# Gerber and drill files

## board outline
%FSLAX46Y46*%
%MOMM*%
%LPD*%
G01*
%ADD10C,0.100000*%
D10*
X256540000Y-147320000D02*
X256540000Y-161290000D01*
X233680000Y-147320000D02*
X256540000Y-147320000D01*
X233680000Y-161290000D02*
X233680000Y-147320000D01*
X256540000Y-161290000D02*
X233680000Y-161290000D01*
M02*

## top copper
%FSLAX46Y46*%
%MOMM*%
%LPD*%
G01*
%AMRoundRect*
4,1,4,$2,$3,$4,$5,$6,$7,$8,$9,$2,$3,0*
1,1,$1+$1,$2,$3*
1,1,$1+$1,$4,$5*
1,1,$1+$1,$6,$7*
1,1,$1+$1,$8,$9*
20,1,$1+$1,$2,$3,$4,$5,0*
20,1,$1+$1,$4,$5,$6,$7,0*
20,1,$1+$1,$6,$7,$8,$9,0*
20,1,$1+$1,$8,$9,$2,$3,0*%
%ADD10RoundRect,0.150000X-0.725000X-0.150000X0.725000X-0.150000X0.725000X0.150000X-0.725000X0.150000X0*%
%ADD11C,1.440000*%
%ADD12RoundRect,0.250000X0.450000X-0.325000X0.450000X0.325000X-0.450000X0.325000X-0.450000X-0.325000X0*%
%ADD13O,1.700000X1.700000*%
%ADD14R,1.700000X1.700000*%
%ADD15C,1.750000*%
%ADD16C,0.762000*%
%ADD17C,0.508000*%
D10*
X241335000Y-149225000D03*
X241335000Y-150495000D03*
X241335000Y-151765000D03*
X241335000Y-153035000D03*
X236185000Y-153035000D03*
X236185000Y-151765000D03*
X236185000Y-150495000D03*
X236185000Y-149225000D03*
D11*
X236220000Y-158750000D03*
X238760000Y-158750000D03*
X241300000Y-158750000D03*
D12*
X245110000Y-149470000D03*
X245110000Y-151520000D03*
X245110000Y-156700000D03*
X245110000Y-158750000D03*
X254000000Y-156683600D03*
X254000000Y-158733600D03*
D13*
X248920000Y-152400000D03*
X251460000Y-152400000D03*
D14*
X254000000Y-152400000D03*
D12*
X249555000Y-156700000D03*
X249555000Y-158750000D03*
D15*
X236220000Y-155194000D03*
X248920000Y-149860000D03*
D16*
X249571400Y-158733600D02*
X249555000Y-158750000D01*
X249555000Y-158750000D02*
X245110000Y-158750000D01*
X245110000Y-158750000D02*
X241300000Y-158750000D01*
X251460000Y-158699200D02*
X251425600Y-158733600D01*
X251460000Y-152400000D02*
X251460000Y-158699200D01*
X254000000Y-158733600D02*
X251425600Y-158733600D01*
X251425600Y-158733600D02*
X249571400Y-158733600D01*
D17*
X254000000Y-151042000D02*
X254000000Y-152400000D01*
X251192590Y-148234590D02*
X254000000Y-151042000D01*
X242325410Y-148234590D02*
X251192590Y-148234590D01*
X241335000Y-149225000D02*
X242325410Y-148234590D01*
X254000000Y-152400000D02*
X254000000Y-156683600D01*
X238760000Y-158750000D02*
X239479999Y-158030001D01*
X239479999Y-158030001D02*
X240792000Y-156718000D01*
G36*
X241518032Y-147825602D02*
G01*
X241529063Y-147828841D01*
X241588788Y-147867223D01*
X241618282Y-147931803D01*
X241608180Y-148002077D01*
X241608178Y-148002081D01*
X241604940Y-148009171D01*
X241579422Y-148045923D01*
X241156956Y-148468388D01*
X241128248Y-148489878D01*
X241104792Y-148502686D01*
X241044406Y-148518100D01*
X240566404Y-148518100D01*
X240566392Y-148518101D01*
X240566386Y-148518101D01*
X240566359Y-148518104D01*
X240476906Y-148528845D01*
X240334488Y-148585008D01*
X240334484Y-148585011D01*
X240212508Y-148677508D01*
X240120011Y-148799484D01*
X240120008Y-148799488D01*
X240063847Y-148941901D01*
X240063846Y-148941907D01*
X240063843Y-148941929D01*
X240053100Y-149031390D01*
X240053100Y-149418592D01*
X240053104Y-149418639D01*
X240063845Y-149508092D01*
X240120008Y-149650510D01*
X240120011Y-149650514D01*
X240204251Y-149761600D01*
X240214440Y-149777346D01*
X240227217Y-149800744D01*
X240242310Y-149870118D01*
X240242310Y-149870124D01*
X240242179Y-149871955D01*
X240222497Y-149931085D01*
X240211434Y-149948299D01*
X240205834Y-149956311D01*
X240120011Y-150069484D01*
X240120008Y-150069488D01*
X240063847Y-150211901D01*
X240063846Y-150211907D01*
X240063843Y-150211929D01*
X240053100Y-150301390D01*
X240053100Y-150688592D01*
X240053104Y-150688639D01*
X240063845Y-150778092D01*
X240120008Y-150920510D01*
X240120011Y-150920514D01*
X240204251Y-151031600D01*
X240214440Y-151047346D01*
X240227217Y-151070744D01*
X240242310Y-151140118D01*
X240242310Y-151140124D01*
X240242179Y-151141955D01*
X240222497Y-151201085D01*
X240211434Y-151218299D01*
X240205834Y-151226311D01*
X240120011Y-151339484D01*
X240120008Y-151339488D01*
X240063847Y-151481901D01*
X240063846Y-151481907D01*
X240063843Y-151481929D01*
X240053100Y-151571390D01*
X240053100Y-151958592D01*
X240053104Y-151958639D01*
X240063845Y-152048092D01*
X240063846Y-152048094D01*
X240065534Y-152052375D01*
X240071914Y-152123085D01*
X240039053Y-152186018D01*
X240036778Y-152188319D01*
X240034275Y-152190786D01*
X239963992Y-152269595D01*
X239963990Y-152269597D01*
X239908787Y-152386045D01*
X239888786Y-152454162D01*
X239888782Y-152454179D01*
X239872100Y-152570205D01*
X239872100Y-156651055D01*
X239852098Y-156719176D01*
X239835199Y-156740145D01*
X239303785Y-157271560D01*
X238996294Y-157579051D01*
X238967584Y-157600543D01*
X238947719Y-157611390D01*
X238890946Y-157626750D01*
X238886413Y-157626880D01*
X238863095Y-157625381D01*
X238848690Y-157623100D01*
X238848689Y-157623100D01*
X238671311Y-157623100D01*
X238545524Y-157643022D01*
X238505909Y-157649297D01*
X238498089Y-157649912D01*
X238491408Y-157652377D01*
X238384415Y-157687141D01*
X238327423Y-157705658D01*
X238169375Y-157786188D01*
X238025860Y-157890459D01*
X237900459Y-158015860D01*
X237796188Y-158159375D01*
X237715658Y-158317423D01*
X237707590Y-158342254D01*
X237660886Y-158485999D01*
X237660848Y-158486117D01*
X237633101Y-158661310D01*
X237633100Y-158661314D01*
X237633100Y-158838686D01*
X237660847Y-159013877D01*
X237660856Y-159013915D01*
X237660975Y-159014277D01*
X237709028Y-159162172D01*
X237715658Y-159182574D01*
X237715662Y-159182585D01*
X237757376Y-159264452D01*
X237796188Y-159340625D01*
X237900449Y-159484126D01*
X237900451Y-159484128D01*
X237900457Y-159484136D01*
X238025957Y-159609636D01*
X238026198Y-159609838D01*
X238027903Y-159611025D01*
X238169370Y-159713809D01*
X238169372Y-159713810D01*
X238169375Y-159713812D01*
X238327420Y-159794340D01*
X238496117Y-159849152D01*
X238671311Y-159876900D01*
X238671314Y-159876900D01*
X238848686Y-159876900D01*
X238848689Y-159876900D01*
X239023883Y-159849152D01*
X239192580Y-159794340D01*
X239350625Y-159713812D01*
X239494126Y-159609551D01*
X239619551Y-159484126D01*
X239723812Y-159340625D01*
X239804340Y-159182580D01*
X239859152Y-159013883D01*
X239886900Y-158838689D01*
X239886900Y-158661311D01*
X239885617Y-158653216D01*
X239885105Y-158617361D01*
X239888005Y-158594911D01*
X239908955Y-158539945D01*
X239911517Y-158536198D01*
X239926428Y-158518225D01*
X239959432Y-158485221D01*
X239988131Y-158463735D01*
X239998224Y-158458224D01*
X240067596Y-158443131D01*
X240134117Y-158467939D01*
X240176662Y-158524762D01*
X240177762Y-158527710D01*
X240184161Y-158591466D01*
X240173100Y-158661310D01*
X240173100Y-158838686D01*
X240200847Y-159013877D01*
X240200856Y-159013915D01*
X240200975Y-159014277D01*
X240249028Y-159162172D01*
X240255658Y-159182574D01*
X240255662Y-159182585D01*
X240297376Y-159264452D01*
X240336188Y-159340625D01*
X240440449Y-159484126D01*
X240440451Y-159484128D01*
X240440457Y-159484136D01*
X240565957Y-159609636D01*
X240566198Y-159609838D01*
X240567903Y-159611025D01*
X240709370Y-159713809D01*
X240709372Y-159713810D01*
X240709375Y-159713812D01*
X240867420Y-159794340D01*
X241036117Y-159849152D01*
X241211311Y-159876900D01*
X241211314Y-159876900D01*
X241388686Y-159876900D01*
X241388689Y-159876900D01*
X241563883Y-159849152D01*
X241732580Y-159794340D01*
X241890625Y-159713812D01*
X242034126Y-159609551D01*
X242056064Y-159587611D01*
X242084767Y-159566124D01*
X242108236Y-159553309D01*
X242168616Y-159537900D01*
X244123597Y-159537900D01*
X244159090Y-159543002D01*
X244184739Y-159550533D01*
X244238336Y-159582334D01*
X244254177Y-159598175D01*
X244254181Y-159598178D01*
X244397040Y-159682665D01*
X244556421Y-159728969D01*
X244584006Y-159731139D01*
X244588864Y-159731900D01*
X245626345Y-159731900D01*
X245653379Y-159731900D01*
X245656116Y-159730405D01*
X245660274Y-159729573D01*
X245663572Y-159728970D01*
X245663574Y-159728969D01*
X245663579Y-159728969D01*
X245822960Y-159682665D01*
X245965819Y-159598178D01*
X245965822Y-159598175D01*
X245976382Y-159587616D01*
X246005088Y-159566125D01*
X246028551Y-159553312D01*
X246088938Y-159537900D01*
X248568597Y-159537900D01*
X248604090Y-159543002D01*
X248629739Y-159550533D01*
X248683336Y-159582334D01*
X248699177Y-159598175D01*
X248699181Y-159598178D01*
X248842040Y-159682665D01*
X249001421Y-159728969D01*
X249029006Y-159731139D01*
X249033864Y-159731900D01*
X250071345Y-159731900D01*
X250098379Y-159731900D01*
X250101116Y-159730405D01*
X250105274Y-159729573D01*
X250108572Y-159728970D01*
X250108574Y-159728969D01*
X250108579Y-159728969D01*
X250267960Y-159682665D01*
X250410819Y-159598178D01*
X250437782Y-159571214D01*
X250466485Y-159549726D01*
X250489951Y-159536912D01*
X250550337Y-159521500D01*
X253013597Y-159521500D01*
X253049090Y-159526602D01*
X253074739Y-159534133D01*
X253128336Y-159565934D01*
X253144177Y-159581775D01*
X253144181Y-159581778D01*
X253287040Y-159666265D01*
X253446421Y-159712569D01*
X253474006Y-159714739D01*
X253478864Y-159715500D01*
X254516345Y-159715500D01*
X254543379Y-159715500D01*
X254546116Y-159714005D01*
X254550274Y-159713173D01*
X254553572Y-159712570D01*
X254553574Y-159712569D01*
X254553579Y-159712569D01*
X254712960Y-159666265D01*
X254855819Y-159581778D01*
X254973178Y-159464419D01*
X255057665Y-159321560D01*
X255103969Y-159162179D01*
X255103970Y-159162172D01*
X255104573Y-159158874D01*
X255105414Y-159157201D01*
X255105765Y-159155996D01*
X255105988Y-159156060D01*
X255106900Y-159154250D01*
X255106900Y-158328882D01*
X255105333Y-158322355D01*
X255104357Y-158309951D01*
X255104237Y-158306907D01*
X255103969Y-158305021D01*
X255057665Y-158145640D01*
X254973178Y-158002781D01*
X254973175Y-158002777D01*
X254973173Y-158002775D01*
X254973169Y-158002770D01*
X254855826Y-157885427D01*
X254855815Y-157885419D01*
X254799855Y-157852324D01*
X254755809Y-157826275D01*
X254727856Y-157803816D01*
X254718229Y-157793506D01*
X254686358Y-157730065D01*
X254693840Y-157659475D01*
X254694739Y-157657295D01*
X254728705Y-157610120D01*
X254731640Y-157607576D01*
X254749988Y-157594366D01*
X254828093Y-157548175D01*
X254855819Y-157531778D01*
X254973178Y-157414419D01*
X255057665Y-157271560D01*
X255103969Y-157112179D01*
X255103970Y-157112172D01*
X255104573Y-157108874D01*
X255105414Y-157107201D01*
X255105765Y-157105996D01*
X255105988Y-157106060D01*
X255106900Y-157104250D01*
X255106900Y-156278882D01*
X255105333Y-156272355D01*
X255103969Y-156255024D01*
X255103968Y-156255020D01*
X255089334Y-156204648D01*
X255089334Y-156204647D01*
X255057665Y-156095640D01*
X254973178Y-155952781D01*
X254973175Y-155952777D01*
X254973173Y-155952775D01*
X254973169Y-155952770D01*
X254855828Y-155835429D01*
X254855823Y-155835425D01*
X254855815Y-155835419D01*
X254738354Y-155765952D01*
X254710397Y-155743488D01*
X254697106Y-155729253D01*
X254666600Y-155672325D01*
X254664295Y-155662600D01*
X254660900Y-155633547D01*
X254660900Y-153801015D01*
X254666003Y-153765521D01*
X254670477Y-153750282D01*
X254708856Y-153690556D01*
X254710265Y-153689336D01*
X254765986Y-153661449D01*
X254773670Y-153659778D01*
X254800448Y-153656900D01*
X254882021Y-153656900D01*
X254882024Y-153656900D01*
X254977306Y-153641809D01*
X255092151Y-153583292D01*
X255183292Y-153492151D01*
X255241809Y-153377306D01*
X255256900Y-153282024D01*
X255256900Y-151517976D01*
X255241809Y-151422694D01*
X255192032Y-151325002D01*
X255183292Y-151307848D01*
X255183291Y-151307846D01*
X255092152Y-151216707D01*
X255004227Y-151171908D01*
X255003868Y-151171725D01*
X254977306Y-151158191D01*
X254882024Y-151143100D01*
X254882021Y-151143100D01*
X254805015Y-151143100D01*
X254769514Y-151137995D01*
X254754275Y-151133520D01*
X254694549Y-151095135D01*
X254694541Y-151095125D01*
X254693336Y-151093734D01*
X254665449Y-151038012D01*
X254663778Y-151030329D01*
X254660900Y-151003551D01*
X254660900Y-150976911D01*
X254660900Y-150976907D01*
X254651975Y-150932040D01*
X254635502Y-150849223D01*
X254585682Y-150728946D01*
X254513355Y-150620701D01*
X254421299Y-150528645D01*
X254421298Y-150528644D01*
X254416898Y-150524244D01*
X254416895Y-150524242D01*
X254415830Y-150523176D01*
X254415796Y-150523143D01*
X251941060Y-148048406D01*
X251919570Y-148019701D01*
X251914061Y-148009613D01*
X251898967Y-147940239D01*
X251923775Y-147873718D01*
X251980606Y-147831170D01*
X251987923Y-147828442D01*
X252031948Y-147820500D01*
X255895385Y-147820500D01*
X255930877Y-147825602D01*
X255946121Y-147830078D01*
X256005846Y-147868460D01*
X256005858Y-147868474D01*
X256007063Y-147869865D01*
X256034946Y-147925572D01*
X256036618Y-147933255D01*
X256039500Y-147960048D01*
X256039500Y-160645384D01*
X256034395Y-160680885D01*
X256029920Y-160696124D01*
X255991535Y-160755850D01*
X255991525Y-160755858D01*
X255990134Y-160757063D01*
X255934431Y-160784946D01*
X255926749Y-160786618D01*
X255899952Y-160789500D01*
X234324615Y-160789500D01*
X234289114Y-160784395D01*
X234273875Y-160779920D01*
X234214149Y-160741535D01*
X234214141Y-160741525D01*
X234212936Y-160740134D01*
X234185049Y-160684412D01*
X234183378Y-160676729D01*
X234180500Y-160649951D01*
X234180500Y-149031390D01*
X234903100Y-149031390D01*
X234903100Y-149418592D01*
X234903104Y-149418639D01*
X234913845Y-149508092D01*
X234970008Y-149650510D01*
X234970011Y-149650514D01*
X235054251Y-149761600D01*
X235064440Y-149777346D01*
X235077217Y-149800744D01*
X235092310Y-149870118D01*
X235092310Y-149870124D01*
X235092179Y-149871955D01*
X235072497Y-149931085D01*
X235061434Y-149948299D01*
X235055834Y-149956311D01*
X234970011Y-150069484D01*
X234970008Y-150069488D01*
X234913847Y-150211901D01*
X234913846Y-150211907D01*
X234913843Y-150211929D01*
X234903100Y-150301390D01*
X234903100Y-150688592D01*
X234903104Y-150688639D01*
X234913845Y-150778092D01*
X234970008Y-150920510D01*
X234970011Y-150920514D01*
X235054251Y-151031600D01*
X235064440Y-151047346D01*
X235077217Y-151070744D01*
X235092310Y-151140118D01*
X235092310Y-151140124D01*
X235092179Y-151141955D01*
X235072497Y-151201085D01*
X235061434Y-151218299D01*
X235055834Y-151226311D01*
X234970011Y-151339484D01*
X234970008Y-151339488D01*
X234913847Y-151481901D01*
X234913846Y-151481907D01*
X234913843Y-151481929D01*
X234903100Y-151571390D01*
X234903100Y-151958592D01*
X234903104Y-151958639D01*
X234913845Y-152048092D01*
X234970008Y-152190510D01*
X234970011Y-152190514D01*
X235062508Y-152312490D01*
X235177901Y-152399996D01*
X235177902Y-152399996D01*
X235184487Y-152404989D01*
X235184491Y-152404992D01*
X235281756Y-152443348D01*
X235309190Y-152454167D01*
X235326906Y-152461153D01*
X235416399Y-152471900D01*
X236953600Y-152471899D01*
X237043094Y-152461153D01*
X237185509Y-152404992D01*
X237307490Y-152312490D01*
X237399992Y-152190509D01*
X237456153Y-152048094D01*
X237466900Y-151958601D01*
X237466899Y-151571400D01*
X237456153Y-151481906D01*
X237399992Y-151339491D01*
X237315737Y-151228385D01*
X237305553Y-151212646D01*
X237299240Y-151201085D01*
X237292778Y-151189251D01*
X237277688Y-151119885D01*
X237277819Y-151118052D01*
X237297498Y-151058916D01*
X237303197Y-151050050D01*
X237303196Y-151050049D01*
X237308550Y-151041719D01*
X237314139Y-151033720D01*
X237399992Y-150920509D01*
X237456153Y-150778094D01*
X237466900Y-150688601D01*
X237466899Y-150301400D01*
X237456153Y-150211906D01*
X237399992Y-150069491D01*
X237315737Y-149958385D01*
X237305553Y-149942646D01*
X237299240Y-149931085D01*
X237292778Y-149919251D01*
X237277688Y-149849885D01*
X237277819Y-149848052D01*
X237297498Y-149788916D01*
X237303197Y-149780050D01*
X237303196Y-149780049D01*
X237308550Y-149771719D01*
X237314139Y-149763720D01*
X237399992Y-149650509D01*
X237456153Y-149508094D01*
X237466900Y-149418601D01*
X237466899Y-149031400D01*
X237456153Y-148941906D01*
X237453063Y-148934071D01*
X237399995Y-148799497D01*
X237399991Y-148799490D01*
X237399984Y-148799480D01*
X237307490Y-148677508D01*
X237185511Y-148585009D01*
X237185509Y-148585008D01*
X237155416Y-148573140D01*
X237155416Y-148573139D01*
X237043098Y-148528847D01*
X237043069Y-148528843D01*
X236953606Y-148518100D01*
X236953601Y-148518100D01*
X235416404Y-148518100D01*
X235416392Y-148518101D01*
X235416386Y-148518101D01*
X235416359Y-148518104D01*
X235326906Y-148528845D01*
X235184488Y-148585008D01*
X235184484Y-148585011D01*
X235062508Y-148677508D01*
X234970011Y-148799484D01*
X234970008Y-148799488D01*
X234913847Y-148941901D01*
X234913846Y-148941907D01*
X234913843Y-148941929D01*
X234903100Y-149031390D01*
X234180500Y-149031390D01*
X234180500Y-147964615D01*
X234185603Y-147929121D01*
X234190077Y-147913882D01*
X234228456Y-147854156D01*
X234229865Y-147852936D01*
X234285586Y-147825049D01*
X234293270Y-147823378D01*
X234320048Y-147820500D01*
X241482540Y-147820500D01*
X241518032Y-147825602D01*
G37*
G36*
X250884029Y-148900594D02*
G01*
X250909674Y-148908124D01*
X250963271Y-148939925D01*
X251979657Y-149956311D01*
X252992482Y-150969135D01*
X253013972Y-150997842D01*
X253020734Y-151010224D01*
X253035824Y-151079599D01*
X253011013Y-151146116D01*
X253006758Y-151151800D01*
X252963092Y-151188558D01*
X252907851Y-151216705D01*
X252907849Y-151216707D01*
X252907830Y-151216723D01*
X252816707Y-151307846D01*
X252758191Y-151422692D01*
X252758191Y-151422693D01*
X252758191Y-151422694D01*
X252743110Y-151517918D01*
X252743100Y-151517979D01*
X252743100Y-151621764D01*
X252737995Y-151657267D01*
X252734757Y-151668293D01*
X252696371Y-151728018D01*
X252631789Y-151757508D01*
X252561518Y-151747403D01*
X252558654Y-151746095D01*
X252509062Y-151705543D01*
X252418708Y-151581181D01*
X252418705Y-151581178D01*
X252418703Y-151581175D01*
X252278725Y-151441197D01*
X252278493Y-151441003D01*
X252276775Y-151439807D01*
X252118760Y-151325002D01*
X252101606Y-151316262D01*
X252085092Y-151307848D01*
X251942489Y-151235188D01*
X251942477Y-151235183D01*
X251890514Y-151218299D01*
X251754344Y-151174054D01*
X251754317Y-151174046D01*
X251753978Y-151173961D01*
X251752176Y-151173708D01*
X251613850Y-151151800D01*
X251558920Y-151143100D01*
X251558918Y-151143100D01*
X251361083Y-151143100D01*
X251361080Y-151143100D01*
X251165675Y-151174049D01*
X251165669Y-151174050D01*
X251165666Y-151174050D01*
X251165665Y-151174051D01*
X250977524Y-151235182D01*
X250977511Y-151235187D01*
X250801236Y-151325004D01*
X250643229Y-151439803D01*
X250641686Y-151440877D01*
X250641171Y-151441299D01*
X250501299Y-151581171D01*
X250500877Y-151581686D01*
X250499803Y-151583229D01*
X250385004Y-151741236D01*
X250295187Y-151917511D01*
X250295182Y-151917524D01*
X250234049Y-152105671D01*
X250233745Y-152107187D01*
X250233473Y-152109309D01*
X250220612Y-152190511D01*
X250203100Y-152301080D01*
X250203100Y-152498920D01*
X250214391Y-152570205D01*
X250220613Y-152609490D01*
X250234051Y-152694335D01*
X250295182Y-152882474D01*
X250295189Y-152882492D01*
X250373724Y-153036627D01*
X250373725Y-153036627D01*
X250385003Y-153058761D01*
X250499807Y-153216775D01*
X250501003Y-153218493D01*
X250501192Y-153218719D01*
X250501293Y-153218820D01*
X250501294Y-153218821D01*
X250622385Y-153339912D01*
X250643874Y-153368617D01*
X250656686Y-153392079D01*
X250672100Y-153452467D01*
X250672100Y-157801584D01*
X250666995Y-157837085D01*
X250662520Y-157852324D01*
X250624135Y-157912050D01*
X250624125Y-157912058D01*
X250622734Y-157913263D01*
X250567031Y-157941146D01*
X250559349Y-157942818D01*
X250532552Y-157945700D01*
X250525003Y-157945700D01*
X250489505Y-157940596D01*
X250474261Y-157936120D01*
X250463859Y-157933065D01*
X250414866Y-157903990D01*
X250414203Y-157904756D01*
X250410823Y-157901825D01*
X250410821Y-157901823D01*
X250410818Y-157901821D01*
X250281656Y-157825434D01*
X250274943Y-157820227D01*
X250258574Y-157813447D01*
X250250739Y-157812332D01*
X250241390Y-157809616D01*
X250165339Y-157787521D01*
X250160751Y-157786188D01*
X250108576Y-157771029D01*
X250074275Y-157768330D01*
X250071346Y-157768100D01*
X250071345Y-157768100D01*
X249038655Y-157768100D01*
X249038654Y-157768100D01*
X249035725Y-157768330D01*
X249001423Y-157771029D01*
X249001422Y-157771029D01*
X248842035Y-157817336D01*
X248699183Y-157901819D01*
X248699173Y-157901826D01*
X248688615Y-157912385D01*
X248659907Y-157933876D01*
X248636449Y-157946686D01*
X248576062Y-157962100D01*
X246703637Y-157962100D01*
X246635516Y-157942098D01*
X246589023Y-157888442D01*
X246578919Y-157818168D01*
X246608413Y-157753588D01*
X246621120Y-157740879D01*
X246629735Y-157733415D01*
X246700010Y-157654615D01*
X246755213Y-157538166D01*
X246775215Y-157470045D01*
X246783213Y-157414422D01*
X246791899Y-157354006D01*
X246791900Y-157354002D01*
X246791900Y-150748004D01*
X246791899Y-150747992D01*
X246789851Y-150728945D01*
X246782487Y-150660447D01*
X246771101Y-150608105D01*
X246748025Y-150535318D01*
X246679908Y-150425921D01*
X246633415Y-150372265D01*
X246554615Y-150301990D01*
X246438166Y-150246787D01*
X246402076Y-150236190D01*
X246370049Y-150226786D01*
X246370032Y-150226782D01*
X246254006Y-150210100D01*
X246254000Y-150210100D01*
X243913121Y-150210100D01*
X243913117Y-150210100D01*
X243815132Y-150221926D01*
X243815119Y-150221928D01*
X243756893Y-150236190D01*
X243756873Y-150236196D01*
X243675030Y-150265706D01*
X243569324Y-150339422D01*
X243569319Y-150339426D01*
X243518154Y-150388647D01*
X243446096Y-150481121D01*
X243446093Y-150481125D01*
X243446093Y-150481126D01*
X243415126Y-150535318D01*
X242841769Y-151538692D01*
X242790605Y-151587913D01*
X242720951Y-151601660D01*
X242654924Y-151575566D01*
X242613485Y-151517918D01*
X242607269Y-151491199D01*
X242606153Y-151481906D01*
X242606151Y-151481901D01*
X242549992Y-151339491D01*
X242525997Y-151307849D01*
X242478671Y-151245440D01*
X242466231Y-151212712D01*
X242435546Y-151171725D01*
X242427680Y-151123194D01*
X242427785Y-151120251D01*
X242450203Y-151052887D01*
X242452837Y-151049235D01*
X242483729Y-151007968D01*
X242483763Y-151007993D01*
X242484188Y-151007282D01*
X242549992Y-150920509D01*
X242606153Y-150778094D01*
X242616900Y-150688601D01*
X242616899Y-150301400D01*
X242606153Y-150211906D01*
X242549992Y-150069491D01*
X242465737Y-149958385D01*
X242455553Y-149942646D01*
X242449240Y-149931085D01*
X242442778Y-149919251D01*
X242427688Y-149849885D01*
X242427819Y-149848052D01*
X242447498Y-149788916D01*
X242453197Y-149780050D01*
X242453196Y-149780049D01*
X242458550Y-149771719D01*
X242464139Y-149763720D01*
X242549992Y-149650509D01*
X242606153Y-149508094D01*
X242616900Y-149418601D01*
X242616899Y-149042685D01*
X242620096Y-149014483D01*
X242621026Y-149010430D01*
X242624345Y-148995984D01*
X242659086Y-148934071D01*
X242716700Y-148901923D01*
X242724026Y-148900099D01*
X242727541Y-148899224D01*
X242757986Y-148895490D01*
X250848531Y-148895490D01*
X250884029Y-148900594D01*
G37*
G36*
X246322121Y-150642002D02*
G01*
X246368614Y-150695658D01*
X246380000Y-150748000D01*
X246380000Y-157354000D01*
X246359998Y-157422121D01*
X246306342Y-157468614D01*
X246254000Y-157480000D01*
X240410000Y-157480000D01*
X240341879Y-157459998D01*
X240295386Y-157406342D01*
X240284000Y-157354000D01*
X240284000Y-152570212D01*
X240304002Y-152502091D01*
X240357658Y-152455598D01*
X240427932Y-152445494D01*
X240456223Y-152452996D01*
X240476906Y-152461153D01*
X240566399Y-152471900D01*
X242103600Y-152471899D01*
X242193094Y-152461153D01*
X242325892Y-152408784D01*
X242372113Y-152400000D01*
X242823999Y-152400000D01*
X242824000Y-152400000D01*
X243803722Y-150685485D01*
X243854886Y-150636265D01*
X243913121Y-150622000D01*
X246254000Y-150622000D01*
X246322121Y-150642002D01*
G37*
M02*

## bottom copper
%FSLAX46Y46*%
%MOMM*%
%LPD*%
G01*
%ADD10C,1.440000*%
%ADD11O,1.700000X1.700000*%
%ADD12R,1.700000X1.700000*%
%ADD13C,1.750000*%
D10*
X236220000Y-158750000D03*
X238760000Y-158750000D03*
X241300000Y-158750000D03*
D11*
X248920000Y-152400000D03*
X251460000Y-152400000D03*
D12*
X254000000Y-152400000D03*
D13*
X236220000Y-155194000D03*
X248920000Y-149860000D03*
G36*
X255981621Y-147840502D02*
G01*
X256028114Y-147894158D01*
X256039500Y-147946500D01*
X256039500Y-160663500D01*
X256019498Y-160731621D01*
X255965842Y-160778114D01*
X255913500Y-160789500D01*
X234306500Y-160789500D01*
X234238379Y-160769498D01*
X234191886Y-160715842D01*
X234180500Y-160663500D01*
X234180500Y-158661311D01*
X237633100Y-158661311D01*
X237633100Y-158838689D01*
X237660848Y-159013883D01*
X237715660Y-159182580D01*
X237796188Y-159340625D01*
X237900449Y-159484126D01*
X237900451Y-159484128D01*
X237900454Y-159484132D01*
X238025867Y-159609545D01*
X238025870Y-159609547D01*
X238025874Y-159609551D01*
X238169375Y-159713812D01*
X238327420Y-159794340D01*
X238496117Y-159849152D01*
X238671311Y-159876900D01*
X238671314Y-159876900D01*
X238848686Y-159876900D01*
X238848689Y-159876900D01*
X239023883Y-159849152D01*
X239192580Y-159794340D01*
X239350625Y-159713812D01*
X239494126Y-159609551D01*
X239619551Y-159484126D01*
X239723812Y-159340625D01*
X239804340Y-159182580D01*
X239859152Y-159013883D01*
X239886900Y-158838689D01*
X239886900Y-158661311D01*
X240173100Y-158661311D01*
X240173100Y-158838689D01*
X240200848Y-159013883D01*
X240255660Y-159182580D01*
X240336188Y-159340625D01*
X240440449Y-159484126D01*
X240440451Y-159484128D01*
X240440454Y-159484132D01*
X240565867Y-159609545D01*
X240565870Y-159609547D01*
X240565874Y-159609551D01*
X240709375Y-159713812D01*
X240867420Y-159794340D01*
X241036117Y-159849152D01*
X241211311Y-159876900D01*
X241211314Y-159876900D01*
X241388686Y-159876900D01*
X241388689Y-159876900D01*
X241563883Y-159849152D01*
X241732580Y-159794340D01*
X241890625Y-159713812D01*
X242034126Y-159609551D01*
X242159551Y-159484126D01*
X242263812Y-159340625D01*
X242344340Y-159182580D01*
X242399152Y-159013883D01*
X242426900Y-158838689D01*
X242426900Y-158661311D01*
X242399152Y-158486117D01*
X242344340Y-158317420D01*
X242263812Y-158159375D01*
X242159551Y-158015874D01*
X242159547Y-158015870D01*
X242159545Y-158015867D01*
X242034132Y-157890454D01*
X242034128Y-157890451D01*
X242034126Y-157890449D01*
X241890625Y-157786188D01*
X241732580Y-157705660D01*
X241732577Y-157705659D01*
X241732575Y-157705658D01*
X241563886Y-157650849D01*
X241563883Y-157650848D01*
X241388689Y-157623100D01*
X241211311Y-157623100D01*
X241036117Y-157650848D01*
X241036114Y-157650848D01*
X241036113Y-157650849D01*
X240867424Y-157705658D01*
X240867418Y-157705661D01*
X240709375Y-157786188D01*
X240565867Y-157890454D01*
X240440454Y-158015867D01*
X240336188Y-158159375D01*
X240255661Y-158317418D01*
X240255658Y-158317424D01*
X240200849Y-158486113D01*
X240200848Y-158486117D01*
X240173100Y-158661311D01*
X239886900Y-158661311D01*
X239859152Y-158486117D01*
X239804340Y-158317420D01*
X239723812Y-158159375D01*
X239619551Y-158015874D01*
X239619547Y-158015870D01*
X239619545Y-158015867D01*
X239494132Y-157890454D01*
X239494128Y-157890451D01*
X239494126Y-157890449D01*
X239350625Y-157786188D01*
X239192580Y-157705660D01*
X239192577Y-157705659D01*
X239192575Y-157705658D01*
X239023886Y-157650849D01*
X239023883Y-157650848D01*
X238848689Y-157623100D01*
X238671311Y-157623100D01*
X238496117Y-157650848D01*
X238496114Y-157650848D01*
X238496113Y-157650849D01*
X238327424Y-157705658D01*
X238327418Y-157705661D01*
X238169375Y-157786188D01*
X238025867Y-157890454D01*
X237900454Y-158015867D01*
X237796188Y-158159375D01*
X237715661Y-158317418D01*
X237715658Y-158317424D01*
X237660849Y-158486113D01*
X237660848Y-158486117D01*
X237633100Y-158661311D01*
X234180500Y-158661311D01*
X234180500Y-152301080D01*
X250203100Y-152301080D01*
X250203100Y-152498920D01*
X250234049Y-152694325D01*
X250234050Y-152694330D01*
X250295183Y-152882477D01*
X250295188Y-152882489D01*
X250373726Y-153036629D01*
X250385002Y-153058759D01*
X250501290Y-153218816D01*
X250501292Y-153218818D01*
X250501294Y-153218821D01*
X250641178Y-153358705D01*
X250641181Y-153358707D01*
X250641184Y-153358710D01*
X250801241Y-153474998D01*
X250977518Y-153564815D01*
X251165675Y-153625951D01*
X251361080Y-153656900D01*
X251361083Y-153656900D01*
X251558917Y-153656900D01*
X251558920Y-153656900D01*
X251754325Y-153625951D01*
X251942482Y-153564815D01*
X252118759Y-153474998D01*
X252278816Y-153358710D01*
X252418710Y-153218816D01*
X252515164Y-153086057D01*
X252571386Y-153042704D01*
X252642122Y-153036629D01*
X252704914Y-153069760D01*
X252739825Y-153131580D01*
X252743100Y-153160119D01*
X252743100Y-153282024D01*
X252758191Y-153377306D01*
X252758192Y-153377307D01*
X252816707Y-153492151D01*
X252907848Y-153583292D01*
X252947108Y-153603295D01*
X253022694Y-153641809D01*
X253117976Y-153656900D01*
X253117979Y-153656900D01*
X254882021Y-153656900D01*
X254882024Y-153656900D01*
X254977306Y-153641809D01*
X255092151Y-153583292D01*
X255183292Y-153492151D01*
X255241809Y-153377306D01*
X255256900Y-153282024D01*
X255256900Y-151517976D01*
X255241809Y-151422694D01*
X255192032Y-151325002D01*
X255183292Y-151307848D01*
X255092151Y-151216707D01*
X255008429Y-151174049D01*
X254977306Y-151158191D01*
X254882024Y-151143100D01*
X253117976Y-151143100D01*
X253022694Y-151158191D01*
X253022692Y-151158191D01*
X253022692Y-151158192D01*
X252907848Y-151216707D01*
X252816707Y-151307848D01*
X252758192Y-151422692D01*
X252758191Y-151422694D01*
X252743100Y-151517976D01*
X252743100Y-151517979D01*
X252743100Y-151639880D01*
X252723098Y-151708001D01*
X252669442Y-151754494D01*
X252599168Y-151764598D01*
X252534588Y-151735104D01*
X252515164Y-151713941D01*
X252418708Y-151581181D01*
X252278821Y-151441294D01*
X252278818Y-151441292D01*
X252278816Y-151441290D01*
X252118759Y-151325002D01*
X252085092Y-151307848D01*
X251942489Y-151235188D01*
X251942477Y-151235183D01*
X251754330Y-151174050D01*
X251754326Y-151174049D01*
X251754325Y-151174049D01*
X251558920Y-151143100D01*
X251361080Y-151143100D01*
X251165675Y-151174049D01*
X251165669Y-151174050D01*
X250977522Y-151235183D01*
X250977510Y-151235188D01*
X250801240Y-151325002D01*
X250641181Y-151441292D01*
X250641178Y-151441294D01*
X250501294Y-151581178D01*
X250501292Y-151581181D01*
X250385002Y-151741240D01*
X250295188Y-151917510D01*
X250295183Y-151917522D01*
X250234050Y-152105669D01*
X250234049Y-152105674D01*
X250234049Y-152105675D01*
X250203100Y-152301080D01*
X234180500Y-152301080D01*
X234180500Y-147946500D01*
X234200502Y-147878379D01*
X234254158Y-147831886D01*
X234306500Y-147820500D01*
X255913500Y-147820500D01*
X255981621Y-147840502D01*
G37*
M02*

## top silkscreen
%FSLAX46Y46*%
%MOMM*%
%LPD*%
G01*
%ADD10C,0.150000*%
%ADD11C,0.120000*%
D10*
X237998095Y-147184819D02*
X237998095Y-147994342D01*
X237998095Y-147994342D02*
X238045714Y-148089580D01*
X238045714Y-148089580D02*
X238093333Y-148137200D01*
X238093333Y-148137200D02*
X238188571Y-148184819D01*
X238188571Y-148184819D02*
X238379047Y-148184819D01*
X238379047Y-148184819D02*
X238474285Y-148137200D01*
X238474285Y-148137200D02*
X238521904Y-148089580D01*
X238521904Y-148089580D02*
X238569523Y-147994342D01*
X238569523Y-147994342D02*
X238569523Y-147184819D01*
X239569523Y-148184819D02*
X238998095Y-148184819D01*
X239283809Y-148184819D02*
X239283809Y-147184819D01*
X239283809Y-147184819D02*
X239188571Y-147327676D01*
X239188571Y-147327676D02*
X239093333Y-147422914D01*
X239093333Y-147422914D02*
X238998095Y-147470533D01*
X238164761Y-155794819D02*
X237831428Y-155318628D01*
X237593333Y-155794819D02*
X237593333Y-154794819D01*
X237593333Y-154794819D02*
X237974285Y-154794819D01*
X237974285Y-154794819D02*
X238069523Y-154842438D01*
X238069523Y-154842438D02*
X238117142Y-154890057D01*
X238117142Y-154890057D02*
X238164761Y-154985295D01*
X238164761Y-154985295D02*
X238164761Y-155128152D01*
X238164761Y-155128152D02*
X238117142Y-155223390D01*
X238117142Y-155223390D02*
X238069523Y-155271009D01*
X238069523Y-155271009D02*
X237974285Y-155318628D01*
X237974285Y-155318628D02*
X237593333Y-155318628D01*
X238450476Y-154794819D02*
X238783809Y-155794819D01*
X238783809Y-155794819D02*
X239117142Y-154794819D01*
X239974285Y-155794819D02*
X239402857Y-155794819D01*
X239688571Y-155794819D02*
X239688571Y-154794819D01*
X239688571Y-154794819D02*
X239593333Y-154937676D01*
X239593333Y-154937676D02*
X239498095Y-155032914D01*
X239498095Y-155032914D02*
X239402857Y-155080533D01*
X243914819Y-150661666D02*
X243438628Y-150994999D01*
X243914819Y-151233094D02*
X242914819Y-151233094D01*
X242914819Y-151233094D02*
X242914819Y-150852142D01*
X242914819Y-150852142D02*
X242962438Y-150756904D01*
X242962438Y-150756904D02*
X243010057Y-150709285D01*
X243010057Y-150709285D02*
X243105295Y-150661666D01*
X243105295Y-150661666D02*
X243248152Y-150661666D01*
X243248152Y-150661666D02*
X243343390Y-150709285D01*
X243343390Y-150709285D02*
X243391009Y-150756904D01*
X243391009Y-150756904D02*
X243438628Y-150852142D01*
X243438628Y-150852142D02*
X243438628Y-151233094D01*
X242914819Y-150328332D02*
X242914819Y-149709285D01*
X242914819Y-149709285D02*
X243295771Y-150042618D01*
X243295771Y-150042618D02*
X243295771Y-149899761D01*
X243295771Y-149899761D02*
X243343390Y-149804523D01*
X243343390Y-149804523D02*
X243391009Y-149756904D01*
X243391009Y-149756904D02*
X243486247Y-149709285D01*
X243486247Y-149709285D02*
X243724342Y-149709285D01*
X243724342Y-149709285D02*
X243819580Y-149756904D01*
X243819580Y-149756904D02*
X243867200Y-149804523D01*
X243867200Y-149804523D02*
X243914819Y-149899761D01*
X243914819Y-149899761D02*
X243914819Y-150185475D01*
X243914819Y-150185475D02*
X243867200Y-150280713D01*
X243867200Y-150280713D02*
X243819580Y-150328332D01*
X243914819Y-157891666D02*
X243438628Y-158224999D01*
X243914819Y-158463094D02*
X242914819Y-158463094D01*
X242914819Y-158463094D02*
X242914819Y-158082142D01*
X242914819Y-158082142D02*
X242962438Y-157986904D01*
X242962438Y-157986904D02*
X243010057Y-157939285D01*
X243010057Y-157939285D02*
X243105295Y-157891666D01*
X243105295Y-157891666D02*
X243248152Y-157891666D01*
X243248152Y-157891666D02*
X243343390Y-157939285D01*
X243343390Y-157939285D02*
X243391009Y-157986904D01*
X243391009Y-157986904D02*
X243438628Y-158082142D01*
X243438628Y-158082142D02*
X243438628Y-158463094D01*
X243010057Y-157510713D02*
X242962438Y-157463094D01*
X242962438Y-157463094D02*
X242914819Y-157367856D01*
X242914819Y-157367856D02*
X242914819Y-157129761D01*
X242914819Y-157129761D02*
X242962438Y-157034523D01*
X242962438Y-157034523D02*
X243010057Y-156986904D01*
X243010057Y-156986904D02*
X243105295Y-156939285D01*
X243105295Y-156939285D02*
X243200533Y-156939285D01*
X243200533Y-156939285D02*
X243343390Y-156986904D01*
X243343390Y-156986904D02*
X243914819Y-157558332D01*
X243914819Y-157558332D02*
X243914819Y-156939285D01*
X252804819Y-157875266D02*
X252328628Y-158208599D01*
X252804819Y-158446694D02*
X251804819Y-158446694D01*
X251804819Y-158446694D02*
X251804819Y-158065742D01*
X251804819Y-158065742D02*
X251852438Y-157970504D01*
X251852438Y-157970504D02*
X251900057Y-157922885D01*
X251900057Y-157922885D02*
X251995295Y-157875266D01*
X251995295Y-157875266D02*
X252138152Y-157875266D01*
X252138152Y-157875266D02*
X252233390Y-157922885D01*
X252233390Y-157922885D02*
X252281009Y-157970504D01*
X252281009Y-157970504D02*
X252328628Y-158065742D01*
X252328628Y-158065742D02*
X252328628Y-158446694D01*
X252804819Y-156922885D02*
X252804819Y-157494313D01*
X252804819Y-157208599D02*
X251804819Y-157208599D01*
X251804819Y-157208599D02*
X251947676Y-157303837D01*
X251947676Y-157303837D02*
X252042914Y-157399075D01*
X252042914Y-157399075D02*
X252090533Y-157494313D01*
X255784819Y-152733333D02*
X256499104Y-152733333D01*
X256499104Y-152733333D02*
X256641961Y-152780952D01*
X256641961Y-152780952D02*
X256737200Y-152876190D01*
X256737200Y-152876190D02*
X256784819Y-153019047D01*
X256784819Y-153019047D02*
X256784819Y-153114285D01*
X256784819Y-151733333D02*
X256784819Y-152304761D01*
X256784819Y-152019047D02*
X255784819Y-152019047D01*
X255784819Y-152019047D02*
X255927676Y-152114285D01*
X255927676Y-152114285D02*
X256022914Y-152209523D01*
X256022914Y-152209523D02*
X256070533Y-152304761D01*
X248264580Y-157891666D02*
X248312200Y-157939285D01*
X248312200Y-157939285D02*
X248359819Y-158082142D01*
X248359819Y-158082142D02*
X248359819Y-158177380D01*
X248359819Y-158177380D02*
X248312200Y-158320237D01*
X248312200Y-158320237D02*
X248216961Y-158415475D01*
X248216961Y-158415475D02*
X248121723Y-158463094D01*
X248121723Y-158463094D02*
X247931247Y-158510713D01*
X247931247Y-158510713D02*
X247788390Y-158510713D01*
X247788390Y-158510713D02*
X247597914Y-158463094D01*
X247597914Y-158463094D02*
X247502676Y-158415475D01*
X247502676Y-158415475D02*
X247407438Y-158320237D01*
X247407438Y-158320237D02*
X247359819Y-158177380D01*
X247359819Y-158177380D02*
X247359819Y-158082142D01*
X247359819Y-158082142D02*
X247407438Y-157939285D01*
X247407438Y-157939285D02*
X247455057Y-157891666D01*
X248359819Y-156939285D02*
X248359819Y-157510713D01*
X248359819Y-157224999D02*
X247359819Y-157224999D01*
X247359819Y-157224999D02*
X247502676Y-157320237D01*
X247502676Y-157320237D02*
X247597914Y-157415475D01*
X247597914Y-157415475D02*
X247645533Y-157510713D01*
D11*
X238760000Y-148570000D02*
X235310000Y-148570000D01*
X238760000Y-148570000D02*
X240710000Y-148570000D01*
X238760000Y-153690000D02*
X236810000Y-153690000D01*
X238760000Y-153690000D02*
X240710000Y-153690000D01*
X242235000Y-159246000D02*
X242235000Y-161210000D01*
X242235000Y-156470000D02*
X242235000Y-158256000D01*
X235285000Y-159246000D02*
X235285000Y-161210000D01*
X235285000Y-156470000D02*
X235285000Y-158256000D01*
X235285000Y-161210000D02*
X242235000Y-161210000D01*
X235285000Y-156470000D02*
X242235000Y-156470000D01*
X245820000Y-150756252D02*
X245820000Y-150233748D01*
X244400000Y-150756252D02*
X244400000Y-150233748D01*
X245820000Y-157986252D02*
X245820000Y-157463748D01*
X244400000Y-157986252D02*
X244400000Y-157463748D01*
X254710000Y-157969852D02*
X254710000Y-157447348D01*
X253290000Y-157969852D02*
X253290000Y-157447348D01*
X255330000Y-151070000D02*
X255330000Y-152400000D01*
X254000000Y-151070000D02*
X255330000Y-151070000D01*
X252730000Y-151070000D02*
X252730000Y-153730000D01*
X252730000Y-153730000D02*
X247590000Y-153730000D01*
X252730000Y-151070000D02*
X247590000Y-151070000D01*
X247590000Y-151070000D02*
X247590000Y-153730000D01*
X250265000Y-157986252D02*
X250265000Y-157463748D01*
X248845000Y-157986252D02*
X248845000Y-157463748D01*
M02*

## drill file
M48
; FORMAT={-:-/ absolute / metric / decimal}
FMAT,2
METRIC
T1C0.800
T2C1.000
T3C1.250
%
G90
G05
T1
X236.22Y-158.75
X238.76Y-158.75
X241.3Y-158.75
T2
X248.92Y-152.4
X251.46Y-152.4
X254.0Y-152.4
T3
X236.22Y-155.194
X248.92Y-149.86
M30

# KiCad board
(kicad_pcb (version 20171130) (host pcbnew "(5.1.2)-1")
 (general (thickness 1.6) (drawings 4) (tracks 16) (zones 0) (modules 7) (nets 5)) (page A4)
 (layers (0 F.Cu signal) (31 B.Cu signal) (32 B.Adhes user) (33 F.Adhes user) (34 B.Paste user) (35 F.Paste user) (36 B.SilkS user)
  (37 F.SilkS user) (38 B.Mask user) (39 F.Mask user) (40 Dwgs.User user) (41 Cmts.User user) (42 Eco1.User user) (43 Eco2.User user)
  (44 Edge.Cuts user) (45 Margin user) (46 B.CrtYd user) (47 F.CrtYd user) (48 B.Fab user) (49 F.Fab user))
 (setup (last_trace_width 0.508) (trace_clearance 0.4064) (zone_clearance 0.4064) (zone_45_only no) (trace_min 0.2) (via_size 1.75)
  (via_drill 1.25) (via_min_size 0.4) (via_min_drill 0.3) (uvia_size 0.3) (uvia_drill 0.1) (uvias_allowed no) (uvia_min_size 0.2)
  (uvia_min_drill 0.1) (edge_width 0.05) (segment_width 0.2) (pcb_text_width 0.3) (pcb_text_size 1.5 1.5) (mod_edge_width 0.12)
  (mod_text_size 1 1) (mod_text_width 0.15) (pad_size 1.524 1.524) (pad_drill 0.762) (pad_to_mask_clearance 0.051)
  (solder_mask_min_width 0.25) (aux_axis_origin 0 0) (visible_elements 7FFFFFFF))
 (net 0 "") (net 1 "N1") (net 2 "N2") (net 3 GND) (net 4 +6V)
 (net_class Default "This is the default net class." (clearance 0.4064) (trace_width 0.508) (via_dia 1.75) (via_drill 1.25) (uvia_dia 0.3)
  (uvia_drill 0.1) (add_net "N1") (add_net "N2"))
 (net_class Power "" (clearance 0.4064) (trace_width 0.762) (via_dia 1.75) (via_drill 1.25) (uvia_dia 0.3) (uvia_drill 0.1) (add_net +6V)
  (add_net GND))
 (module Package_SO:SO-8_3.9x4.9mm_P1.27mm (layer F.Cu) (at 238.76 151.13)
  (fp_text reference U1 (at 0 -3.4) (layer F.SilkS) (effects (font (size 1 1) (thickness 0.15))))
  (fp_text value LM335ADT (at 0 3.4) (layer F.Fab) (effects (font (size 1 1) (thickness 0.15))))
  (fp_line (start 0 -2.56) (end -3.45 -2.56) (layer F.SilkS) (width 0.12))
  (fp_line (start 0 -2.56) (end 1.95 -2.56) (layer F.SilkS) (width 0.12))
  (fp_line (start 0 2.56) (end -1.95 2.56) (layer F.SilkS) (width 0.12))
  (fp_line (start 0 2.56) (end 1.95 2.56) (layer F.SilkS) (width 0.12))
  (pad 8 smd roundrect (at 2.575 -1.905) (size 1.75 0.6) (layers F.Cu F.Paste F.Mask) (roundrect_rratio 0.25) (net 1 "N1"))
  (pad 7 smd roundrect (at 2.575 -0.635) (size 1.75 0.6) (layers F.Cu F.Paste F.Mask) (roundrect_rratio 0.25))
  (pad 6 smd roundrect (at 2.575 0.635) (size 1.75 0.6) (layers F.Cu F.Paste F.Mask) (roundrect_rratio 0.25))
  (pad 5 smd roundrect (at 2.575 1.905) (size 1.75 0.6) (layers F.Cu F.Paste F.Mask) (roundrect_rratio 0.25) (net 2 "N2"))
  (pad 4 smd roundrect (at -2.575 1.905) (size 1.75 0.6) (layers F.Cu F.Paste F.Mask) (roundrect_rratio 0.25) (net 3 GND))
  (pad 3 smd roundrect (at -2.575 0.635) (size 1.75 0.6) (layers F.Cu F.Paste F.Mask) (roundrect_rratio 0.25))
  (pad 2 smd roundrect (at -2.575 -0.635) (size 1.75 0.6) (layers F.Cu F.Paste F.Mask) (roundrect_rratio 0.25))
  (pad 1 smd roundrect (at -2.575 -1.905) (size 1.75 0.6) (layers F.Cu F.Paste F.Mask) (roundrect_rratio 0.25)))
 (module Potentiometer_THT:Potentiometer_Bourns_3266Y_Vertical (layer F.Cu) (at 241.3 158.75)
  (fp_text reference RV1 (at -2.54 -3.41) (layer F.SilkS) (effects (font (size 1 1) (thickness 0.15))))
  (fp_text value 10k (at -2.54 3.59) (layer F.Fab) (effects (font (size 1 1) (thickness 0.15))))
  (fp_line (start 0.935 0.496) (end 0.935 2.46) (layer F.SilkS) (width 0.12))
  (fp_line (start 0.935 -2.28) (end 0.935 -0.494) (layer F.SilkS) (width 0.12))
  (fp_line (start -6.015 0.496) (end -6.015 2.46) (layer F.SilkS) (width 0.12))
  (fp_line (start -6.015 -2.28) (end -6.015 -0.494) (layer F.SilkS) (width 0.12))
  (fp_line (start -6.015 2.46) (end 0.935 2.46) (layer F.SilkS) (width 0.12))
  (fp_line (start -6.015 -2.28) (end 0.935 -2.28) (layer F.SilkS) (width 0.12))
  (pad 3 thru_hole circle (at -5.08 0) (size 1.44 1.44) (drill 0.8) (layers *.Cu *.Mask) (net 3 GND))
  (pad 2 thru_hole circle (at -2.54 0) (size 1.44 1.44) (drill 0.8) (layers *.Cu *.Mask) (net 2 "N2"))
  (pad 1 thru_hole circle (at 0 0) (size 1.44 1.44) (drill 0.8) (layers *.Cu *.Mask) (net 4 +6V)))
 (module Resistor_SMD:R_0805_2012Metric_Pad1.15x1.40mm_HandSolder (layer F.Cu) (at 245.11 150.495 90)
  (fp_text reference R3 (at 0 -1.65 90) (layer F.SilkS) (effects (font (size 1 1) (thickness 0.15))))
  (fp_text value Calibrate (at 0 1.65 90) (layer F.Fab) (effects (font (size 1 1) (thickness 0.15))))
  (fp_line (start -0.261252 0.71) (end 0.261252 0.71) (layer F.SilkS) (width 0.12))
  (fp_line (start -0.261252 -0.71) (end 0.261252 -0.71) (layer F.SilkS) (width 0.12))
  (pad 2 smd roundrect (at 1.025 0 90) (size 1.15 1.4) (layers F.Cu F.Paste F.Mask) (roundrect_rratio 0.217391) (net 3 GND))
  (pad 1 smd roundrect (at -1.025 0 90) (size 1.15 1.4) (layers F.Cu F.Paste F.Mask) (roundrect_rratio 0.217391) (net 2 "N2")))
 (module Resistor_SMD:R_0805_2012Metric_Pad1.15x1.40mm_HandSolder (layer F.Cu) (at 245.11 157.725 90)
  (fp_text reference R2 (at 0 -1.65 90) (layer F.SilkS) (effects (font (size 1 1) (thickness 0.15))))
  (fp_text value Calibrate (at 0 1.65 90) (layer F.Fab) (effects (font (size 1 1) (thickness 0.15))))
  (fp_line (start -0.261252 0.71) (end 0.261252 0.71) (layer F.SilkS) (width 0.12))
  (fp_line (start -0.261252 -0.71) (end 0.261252 -0.71) (layer F.SilkS) (width 0.12))
  (pad 2 smd roundrect (at 1.025 0 90) (size 1.15 1.4) (layers F.Cu F.Paste F.Mask) (roundrect_rratio 0.217391) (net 2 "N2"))
  (pad 1 smd roundrect (at -1.025 0 90) (size 1.15 1.4) (layers F.Cu F.Paste F.Mask) (roundrect_rratio 0.217391) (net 4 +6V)))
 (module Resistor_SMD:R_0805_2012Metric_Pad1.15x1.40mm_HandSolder (layer F.Cu) (at 254 157.7086 90)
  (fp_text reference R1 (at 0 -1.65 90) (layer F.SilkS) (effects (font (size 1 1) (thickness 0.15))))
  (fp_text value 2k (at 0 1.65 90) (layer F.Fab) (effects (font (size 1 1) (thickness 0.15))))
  (fp_line (start -0.261252 0.71) (end 0.261252 0.71) (layer F.SilkS) (width 0.12))
  (fp_line (start -0.261252 -0.71) (end 0.261252 -0.71) (layer F.SilkS) (width 0.12))
  (pad 2 smd roundrect (at 1.025 0 90) (size 1.15 1.4) (layers F.Cu F.Paste F.Mask) (roundrect_rratio 0.217391) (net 1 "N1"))
  (pad 1 smd roundrect (at -1.025 0 90) (size 1.15 1.4) (layers F.Cu F.Paste F.Mask) (roundrect_rratio 0.217391) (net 4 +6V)))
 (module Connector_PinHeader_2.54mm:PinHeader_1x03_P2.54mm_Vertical (layer F.Cu) (at 254 152.4 270)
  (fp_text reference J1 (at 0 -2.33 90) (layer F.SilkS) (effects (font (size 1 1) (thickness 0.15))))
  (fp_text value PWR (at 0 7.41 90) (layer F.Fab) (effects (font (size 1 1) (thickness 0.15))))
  (fp_line (start -1.33 -1.33) (end 0 -1.33) (layer F.SilkS) (width 0.12))
  (fp_line (start -1.33 0) (end -1.33 -1.33) (layer F.SilkS) (width 0.12))
  (fp_line (start -1.33 1.27) (end 1.33 1.27) (layer F.SilkS) (width 0.12))
  (fp_line (start 1.33 1.27) (end 1.33 6.41) (layer F.SilkS) (width 0.12))
  (fp_line (start -1.33 1.27) (end -1.33 6.41) (layer F.SilkS) (width 0.12))
  (fp_line (start -1.33 6.41) (end 1.33 6.41) (layer F.SilkS) (width 0.12))
  (pad 3 thru_hole oval (at 0 5.08 270) (size 1.7 1.7) (drill 1) (layers *.Cu *.Mask) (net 3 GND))
  (pad 2 thru_hole oval (at 0 2.54 270) (size 1.7 1.7) (drill 1) (layers *.Cu *.Mask) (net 4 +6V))
  (pad 1 thru_hole rect (at 0 0 270) (size 1.7 1.7) (drill 1) (layers *.Cu *.Mask) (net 1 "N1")))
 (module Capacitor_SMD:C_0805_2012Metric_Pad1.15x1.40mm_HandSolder (layer F.Cu) (at 249.555 157.725 90)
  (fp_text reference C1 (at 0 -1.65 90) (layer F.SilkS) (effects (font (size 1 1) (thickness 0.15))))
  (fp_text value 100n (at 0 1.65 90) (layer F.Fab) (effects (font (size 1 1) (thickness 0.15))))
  (fp_line (start -0.261252 0.71) (end 0.261252 0.71) (layer F.SilkS) (width 0.12))
  (fp_line (start -0.261252 -0.71) (end 0.261252 -0.71) (layer F.SilkS) (width 0.12))
  (pad 2 smd roundrect (at 1.025 0 90) (size 1.15 1.4) (layers F.Cu F.Paste F.Mask) (roundrect_rratio 0.217391) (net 3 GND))
  (pad 1 smd roundrect (at -1.025 0 90) (size 1.15 1.4) (layers F.Cu F.Paste F.Mask) (roundrect_rratio 0.217391) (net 4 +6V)))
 (gr_line (start 256.54 147.32) (end 256.54 161.29) (layer Edge.Cuts) (width 0.1))
 (gr_line (start 233.68 147.32) (end 256.54 147.32) (layer Edge.Cuts) (width 0.1))
 (gr_line (start 233.68 161.29) (end 233.68 147.32) (layer Edge.Cuts) (width 0.1))
 (gr_line (start 256.54 161.29) (end 233.68 161.29) (layer Edge.Cuts) (width 0.1))
 (via (at 236.22 155.194) (size 1.75) (drill 1.25) (layers F.Cu B.Cu) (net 3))
 (via (at 248.92 149.86) (size 1.75) (drill 1.25) (layers F.Cu B.Cu) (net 3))
 (segment (start 249.5714 158.7336) (end 249.555 158.75) (width 0.762) (layer F.Cu) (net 4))
 (segment (start 249.555 158.75) (end 245.11 158.75) (width 0.762) (layer F.Cu) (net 4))
 (segment (start 245.11 158.75) (end 241.3 158.75) (width 0.762) (layer F.Cu) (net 4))
 (segment (start 251.46 158.6992) (end 251.4256 158.7336) (width 0.762) (layer F.Cu) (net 4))
 (segment (start 251.46 152.4) (end 251.46 158.6992) (width 0.762) (layer F.Cu) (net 4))
 (segment (start 254 158.7336) (end 251.4256 158.7336) (width 0.762) (layer F.Cu) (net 4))
 (segment (start 251.4256 158.7336) (end 249.5714 158.7336) (width 0.762) (layer F.Cu) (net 4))
 (segment (start 254 151.042) (end 254 152.4) (width 0.508) (layer F.Cu) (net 1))
 (segment (start 251.19259 148.23459) (end 254 151.042) (width 0.508) (layer F.Cu) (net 1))
 (segment (start 242.32541 148.23459) (end 251.19259 148.23459) (width 0.508) (layer F.Cu) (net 1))
 (segment (start 241.335 149.225) (end 242.32541 148.23459) (width 0.508) (layer F.Cu) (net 1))
 (segment (start 254 152.4) (end 254 156.6836) (width 0.508) (layer F.Cu) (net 1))
 (segment (start 238.76 158.75) (end 239.479999 158.030001) (width 0.508) (layer F.Cu) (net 2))
 (segment (start 239.479999 158.030001) (end 240.792 156.718) (width 0.508) (layer F.Cu) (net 2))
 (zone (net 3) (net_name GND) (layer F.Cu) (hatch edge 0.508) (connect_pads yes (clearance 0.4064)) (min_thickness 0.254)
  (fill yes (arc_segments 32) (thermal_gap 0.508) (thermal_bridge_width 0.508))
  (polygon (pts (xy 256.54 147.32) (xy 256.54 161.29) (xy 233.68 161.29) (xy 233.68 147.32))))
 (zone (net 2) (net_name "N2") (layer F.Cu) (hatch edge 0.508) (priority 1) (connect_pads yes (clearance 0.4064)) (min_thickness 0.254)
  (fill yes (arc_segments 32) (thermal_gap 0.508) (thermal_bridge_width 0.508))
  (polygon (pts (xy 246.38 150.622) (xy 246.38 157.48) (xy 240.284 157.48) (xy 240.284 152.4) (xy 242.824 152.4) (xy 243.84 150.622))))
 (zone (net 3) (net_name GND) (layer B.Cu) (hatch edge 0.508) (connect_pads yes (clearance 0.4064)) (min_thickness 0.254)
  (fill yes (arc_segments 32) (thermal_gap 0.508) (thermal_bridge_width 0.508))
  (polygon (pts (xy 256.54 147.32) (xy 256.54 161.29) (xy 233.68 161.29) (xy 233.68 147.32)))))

